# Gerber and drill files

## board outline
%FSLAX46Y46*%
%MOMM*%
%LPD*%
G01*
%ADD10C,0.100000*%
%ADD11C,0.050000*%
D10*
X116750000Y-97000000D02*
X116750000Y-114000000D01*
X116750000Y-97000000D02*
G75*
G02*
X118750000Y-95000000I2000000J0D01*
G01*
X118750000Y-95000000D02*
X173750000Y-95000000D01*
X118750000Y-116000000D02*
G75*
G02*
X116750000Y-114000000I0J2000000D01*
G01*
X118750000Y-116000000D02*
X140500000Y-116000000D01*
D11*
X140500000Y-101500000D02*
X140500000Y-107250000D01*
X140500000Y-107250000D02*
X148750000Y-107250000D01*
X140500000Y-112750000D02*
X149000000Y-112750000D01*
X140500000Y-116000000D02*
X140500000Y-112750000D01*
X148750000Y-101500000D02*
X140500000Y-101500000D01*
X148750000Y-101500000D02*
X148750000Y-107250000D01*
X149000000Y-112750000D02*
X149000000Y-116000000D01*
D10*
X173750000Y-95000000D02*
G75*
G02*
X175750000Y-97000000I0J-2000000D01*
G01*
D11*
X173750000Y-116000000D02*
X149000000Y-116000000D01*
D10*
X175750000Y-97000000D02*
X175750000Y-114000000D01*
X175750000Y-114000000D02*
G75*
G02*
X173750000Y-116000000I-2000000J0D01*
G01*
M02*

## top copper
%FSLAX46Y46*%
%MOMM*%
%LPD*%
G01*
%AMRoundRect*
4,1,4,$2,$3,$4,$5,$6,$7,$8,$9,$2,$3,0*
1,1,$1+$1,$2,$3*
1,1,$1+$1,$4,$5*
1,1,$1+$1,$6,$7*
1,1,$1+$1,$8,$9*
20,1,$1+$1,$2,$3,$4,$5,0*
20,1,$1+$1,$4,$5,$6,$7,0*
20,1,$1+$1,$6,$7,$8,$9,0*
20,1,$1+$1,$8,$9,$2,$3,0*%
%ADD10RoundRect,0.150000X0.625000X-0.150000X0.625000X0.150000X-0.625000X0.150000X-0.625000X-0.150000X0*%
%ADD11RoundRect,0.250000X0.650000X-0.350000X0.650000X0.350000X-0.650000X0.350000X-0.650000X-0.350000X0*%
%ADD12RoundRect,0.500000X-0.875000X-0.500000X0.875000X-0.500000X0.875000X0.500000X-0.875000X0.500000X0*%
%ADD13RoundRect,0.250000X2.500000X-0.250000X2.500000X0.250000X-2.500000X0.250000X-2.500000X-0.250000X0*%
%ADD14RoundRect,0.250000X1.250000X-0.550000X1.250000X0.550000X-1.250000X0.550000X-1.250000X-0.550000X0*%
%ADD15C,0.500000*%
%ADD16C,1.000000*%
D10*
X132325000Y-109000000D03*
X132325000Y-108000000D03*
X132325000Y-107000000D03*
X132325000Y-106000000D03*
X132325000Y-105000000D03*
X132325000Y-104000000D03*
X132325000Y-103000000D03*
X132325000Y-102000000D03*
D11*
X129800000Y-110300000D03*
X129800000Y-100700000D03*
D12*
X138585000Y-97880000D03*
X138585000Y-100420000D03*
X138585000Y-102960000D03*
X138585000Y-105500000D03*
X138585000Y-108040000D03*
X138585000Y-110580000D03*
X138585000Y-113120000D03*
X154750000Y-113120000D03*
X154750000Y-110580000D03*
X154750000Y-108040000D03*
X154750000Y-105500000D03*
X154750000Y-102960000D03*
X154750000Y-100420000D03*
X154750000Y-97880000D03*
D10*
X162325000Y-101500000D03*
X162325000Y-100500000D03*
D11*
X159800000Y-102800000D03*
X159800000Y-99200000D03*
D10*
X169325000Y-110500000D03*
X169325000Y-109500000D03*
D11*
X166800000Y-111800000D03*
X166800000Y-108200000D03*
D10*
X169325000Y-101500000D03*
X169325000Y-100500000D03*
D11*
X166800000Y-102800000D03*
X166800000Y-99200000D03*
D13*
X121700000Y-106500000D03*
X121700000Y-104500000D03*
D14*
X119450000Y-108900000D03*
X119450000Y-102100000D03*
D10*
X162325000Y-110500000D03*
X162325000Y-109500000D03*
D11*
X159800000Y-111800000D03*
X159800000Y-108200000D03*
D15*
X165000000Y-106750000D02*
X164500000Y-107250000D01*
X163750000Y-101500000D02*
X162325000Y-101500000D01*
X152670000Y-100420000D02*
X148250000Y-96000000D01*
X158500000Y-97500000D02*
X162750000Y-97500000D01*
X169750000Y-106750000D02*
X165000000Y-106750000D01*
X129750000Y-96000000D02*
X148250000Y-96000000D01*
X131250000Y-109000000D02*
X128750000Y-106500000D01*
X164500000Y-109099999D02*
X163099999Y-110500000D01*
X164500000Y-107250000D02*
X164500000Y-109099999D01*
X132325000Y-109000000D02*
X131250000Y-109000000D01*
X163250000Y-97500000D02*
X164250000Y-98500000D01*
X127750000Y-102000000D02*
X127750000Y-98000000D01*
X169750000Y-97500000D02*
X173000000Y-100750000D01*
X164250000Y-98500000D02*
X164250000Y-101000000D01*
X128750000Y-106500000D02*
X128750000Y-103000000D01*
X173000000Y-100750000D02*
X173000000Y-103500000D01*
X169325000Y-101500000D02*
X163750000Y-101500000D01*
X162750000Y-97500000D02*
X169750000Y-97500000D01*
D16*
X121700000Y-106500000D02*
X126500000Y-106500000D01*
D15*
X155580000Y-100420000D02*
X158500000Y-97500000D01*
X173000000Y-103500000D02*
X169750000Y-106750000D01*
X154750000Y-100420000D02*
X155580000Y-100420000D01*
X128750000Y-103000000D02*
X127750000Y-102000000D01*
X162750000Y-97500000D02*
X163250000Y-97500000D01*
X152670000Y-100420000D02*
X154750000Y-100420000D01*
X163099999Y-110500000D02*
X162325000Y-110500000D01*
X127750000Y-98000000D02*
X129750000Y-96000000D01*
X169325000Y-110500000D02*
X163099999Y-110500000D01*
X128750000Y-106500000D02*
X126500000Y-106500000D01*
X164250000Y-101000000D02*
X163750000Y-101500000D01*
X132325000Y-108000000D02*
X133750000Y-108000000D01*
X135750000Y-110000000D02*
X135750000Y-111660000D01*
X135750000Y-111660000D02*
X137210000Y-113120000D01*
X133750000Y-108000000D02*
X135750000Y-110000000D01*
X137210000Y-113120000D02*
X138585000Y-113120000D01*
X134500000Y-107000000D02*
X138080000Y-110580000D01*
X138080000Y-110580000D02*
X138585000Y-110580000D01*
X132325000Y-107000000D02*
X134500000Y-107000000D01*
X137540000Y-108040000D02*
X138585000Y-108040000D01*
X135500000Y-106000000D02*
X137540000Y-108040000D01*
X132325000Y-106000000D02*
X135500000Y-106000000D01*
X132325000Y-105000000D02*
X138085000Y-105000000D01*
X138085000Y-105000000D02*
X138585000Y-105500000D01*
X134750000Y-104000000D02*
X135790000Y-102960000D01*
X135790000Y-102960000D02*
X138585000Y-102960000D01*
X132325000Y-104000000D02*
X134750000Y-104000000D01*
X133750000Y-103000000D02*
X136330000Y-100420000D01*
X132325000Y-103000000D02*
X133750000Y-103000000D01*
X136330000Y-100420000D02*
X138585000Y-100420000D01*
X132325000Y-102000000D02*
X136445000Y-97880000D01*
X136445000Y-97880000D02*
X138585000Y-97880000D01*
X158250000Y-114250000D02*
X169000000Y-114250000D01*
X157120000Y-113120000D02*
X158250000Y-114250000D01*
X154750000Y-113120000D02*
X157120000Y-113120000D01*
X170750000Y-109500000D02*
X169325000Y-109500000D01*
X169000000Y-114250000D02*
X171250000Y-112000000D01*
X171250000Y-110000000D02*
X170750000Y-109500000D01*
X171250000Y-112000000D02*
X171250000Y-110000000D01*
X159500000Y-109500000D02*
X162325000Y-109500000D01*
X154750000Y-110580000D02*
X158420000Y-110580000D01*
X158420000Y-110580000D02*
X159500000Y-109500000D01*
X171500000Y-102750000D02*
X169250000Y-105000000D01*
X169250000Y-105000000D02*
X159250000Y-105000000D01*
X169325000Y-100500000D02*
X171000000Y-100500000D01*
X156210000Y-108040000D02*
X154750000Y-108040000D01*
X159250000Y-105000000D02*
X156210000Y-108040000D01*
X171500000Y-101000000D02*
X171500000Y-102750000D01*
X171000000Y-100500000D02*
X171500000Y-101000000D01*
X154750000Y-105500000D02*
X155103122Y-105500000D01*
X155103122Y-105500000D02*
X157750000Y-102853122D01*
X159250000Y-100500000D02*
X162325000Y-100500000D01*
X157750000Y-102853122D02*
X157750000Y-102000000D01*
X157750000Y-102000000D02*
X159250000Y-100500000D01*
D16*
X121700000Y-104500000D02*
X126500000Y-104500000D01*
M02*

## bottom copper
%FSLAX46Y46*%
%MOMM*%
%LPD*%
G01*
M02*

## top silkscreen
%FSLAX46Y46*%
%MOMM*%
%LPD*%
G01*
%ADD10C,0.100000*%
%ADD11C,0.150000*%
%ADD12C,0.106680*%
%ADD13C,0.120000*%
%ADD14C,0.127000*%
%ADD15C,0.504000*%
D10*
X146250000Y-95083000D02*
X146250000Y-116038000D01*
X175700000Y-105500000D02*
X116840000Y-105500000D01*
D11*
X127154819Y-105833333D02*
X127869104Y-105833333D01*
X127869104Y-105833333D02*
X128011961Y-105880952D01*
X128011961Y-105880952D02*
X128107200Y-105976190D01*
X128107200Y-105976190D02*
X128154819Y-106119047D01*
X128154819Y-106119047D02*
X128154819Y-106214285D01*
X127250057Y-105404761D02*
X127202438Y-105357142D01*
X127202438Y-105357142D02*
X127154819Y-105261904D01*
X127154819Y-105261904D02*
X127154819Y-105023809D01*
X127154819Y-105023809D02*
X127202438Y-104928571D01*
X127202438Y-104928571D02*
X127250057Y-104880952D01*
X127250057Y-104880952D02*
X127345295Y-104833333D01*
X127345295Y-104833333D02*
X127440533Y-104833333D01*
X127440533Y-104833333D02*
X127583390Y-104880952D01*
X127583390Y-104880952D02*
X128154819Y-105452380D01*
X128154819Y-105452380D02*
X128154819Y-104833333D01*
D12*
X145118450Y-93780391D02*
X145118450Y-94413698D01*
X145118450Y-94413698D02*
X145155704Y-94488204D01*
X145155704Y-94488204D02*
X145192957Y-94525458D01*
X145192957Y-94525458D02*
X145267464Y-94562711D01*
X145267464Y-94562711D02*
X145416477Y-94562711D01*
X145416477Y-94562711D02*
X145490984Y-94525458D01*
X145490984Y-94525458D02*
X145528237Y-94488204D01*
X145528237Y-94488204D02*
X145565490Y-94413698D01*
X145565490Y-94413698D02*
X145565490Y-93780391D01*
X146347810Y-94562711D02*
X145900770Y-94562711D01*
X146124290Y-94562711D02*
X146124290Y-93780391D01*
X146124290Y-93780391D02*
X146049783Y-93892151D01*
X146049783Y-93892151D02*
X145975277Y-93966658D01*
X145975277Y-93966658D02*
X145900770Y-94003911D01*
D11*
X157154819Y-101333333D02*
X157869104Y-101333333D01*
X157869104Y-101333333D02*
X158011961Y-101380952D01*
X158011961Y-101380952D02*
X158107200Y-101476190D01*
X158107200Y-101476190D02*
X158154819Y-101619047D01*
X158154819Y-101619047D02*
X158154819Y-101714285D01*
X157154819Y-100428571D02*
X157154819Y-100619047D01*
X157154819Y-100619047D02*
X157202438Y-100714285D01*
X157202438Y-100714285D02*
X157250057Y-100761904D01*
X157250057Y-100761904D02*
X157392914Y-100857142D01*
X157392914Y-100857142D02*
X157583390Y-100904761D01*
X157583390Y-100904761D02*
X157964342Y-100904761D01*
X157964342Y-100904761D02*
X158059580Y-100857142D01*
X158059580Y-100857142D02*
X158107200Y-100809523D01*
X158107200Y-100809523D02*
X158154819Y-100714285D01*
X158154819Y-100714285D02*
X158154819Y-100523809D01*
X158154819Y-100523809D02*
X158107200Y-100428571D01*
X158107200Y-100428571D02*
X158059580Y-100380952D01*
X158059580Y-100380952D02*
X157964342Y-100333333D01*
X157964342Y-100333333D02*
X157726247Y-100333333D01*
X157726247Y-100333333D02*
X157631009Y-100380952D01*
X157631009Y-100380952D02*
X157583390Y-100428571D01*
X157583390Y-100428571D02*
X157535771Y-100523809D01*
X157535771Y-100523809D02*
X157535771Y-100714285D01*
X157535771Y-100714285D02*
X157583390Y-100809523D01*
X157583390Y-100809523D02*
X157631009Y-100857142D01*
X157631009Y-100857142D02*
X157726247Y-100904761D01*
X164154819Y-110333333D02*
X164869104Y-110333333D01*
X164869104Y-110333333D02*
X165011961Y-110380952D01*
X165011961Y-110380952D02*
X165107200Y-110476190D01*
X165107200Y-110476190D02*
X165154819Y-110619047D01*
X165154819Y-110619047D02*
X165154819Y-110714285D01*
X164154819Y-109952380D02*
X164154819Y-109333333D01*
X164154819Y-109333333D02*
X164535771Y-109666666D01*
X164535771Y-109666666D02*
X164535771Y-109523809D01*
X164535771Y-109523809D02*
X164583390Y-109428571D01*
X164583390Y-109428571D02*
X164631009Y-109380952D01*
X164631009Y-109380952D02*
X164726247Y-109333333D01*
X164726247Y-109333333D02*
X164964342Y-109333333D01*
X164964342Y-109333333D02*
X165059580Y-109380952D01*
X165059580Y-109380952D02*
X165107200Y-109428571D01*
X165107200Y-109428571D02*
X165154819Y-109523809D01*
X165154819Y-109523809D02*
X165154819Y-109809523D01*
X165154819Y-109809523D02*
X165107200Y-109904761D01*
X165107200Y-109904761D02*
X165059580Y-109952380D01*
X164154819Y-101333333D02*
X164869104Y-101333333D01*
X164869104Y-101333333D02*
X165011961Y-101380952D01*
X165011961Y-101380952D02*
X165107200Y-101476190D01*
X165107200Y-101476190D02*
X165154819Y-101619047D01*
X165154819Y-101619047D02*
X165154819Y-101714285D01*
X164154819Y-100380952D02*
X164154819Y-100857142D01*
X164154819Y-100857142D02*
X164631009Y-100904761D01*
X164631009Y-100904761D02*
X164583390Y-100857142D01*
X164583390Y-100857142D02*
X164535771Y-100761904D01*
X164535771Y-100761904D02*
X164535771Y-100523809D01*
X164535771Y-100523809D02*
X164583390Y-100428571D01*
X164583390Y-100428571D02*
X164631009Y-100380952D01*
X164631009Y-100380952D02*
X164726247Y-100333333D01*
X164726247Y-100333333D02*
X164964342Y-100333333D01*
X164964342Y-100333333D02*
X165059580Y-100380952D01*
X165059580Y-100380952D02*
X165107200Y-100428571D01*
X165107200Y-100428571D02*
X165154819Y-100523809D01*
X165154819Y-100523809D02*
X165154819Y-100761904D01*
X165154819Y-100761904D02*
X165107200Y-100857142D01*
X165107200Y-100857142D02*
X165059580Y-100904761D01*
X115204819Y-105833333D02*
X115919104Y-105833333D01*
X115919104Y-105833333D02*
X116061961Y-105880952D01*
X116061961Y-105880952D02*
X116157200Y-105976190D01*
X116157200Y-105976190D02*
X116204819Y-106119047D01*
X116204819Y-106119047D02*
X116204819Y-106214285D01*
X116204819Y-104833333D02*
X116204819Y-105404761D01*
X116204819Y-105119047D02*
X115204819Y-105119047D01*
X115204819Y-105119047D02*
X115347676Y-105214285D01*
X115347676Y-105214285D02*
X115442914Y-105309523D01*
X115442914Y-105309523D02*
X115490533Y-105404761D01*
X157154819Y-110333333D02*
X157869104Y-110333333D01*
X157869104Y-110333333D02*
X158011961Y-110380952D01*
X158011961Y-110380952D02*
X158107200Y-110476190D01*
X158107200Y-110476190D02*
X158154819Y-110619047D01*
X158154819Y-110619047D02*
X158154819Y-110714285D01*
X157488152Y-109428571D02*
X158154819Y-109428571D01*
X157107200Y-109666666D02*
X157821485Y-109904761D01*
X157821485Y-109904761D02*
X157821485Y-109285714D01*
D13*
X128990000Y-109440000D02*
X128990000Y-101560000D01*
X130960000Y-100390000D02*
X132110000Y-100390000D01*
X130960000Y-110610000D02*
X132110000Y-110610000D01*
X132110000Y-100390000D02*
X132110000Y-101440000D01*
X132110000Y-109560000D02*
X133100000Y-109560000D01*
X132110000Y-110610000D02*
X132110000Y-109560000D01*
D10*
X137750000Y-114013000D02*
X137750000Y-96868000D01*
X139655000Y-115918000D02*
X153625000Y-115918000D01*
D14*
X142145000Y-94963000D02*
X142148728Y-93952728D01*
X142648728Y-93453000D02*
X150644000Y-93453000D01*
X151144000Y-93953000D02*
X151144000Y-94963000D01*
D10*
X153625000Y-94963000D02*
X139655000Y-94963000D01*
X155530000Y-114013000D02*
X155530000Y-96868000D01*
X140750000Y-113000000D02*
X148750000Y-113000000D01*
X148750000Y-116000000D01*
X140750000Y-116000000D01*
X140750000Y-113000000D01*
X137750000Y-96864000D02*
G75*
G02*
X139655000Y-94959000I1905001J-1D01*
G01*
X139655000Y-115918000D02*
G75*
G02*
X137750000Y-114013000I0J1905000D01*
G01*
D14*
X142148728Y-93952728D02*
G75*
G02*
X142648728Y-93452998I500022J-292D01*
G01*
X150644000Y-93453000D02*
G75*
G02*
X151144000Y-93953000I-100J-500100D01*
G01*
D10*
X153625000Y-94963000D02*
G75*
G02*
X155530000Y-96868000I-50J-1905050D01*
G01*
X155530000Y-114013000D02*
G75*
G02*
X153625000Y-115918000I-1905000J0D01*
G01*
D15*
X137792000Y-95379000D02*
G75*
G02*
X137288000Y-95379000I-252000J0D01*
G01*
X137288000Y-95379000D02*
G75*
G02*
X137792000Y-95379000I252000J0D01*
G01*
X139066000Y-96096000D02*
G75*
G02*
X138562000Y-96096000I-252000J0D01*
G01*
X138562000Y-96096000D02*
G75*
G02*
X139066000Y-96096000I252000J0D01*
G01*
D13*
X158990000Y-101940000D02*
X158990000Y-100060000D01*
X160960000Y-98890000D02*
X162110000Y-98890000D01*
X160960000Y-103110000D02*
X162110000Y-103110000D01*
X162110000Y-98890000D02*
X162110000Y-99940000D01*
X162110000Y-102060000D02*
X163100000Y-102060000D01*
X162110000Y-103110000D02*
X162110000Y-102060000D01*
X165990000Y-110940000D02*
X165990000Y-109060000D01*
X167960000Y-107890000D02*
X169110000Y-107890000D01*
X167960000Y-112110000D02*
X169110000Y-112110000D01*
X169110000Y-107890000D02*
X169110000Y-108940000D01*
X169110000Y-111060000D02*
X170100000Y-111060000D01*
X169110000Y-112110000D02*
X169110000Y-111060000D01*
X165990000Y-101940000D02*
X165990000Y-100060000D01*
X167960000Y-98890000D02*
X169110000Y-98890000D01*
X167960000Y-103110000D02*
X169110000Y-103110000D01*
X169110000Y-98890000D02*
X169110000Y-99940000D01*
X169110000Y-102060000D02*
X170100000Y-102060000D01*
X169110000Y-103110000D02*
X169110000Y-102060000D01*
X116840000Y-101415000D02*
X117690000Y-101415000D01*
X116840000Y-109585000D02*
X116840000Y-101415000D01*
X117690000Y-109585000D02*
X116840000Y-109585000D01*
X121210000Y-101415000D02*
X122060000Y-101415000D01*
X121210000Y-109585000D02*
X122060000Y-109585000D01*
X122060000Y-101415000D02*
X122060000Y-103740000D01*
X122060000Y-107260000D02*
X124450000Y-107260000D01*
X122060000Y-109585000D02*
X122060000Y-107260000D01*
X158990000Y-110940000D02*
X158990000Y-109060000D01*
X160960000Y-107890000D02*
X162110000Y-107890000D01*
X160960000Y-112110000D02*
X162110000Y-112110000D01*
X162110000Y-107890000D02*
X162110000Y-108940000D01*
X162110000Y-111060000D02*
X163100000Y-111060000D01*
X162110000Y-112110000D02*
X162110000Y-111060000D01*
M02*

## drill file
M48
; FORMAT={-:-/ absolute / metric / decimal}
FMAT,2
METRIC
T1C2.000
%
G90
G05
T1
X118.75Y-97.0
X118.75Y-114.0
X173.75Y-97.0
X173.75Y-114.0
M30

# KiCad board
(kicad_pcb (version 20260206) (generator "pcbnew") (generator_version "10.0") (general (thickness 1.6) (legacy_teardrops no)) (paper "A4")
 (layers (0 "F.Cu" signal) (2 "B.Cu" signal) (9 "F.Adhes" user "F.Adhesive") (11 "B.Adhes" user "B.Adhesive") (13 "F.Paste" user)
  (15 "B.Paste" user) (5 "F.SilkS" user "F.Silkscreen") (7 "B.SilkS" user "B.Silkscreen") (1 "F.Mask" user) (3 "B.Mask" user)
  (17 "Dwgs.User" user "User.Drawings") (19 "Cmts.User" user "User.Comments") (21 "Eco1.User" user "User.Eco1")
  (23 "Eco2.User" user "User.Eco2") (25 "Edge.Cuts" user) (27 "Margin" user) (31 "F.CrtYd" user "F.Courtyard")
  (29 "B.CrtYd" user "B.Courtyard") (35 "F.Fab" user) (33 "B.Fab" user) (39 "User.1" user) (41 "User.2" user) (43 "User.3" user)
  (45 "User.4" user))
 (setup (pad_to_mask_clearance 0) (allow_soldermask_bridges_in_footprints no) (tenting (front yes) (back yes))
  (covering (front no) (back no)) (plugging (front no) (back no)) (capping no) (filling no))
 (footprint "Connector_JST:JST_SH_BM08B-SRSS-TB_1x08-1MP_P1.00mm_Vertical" (layer "F.Cu") (at 131 105.5 90)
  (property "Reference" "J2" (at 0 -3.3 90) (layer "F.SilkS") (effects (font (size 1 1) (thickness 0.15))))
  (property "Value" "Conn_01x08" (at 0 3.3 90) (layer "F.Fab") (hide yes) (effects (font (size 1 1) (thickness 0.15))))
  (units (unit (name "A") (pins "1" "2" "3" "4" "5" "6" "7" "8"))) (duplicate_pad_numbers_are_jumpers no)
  (fp_line (start -3.94 -2.01) (end 3.94 -2.01) (stroke (width 0.12) (type solid)) (layer "F.SilkS"))
  (fp_line (start 5.11 -0.04) (end 5.11 1.11) (stroke (width 0.12) (type solid)) (layer "F.SilkS"))
  (fp_line (start -5.11 -0.04) (end -5.11 1.11) (stroke (width 0.12) (type solid)) (layer "F.SilkS"))
  (fp_line (start 5.11 1.11) (end 4.06 1.11) (stroke (width 0.12) (type solid)) (layer "F.SilkS"))
  (fp_line (start -4.06 1.11) (end -4.06 2.1) (stroke (width 0.12) (type solid)) (layer "F.SilkS"))
  (fp_line (start -5.11 1.11) (end -4.06 1.11) (stroke (width 0.12) (type solid)) (layer "F.SilkS"))
  (pad "1" smd roundrect (at -3.5 1.325 90) (size 0.6 1.55) (layers "F.Cu" "F.Mask" "F.Paste") (roundrect_rratio 0.25) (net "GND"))
  (pad "2" smd roundrect (at -2.5 1.325 90) (size 0.6 1.55) (layers "F.Cu" "F.Mask" "F.Paste") (roundrect_rratio 0.25)
   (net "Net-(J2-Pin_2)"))
  (pad "3" smd roundrect (at -1.5 1.325 90) (size 0.6 1.55) (layers "F.Cu" "F.Mask" "F.Paste") (roundrect_rratio 0.25)
   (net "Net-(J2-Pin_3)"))
  (pad "4" smd roundrect (at -0.5 1.325 90) (size 0.6 1.55) (layers "F.Cu" "F.Mask" "F.Paste") (roundrect_rratio 0.25)
   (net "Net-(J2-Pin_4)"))
  (pad "5" smd roundrect (at 0.5 1.325 90) (size 0.6 1.55) (layers "F.Cu" "F.Mask" "F.Paste") (roundrect_rratio 0.25) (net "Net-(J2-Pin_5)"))
  (pad "6" smd roundrect (at 1.5 1.325 90) (size 0.6 1.55) (layers "F.Cu" "F.Mask" "F.Paste") (roundrect_rratio 0.25) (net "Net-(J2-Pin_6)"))
  (pad "7" smd roundrect (at 2.5 1.325 90) (size 0.6 1.55) (layers "F.Cu" "F.Mask" "F.Paste") (roundrect_rratio 0.25) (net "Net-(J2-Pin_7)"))
  (pad "8" smd roundrect (at 3.5 1.325 90) (size 0.6 1.55) (layers "F.Cu" "F.Mask" "F.Paste") (roundrect_rratio 0.25) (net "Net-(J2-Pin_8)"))
  (pad "MP" smd roundrect (at -4.8 -1.2 90) (size 1.2 1.8) (layers "F.Cu" "F.Mask" "F.Paste") (roundrect_rratio 0.208333))
  (pad "MP" smd roundrect (at 4.8 -1.2 90) (size 1.2 1.8) (layers "F.Cu" "F.Mask" "F.Paste") (roundrect_rratio 0.208333)))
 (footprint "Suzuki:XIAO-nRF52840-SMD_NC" (layer "F.Cu") (at 137.75 116)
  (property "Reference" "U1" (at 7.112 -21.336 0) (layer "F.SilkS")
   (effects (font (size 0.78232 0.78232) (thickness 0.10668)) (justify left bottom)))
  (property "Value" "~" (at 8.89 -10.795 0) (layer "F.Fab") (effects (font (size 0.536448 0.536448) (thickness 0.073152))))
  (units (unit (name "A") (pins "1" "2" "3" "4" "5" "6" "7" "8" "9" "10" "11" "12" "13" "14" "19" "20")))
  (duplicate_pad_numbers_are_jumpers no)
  (fp_line (start 0 -1.987) (end 0 -19.132) (stroke (width 0.1) (type solid)) (layer "F.SilkS"))
  (fp_line (start 1.905 -0.082) (end 15.875 -0.082) (stroke (width 0.1) (type solid)) (layer "F.SilkS"))
  (fp_line (start 4.395 -21.037) (end 4.398728 -22.047272) (stroke (width 0.127) (type solid)) (layer "F.SilkS"))
  (fp_line (start 4.898728 -22.547) (end 12.894 -22.547) (stroke (width 0.127) (type solid)) (layer "F.SilkS"))
  (fp_line (start 13.394 -22.047) (end 13.394 -21.037) (stroke (width 0.127) (type solid)) (layer "F.SilkS"))
  (fp_line (start 15.875 -21.037) (end 1.905 -21.037) (stroke (width 0.1) (type solid)) (layer "F.SilkS"))
  (fp_line (start 17.78 -1.987) (end 17.78 -19.132) (stroke (width 0.1) (type solid)) (layer "F.SilkS"))
  (fp_rect (start 3 -3) (end 11 0) (stroke (width 0.1) (type default)) (fill no) (layer "F.SilkS"))
  (fp_arc (start 0 -19.136) (mid 0.557962 -20.483038) (end 1.905 -21.041) (stroke (width 0.1) (type solid)) (layer "F.SilkS"))
  (fp_arc (start 1.905 -0.082) (mid 0.557962 -0.639962) (end 0 -1.987) (stroke (width 0.1) (type solid)) (layer "F.SilkS"))
  (fp_arc (start 4.398728 -22.047272) (mid 4.545276 -22.400644) (end 4.898728 -22.547) (stroke (width 0.127) (type default))
   (layer "F.SilkS"))
  (fp_arc (start 12.894 -22.547) (mid 13.247531 -22.400546) (end 13.394 -22.047) (stroke (width 0.127) (type default)) (layer "F.SilkS"))
  (fp_arc (start 15.875 -21.037) (mid 17.222016 -20.479031) (end 17.78 -19.132) (stroke (width 0.1) (type solid)) (layer "F.SilkS"))
  (fp_arc (start 17.78 -1.987) (mid 17.222038 -0.639961) (end 15.875 -0.082) (stroke (width 0.1) (type solid)) (layer "F.SilkS"))
  (fp_circle (center -0.21 -20.621) (end -0.21 -20.875) (stroke (width 0.5) (type solid)) (fill yes) (layer "F.SilkS"))
  (fp_circle (center 1.064 -19.904) (end 1.064 -20.158) (stroke (width 0.5) (type solid)) (fill yes) (layer "F.SilkS"))
  (pad "1" smd roundrect (at 0.835 -18.12) (size 2.75 2) (layers "F.Cu" "F.Mask" "F.Paste") (roundrect_rratio 0.25) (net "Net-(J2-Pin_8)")
   (solder_mask_margin 0.0508) (thermal_bridge_angle 45))
  (pad "2" smd roundrect (at 0.835 -15.58) (size 2.75 2) (layers "F.Cu" "F.Mask" "F.Paste") (roundrect_rratio 0.25) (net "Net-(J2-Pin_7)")
   (solder_mask_margin 0.0508) (thermal_bridge_angle 45))
  (pad "3" smd roundrect (at 0.835 -13.04) (size 2.75 2) (layers "F.Cu" "F.Mask" "F.Paste") (roundrect_rratio 0.25) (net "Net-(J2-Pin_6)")
   (solder_mask_margin 0.0508) (thermal_bridge_angle 45))
  (pad "4" smd roundrect (at 0.835 -10.5) (size 2.75 2) (layers "F.Cu" "F.Mask" "F.Paste") (roundrect_rratio 0.25) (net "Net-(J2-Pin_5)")
   (solder_mask_margin 0.0508) (thermal_bridge_angle 45))
  (pad "5" smd roundrect (at 0.835 -7.96) (size 2.75 2) (layers "F.Cu" "F.Mask" "F.Paste") (roundrect_rratio 0.25) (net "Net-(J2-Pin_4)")
   (solder_mask_margin 0.0508) (thermal_bridge_angle 45))
  (pad "6" smd roundrect (at 0.835 -5.42) (size 2.75 2) (layers "F.Cu" "F.Mask" "F.Paste") (roundrect_rratio 0.25) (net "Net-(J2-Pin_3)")
   (solder_mask_margin 0.0508) (thermal_bridge_angle 45))
  (pad "7" smd roundrect (at 0.835 -2.88) (size 2.75 2) (layers "F.Cu" "F.Mask" "F.Paste") (roundrect_rratio 0.25) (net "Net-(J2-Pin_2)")
   (solder_mask_margin 0.0508) (thermal_bridge_angle 45))
  (pad "8" smd roundrect (at 17 -2.88) (size 2.75 2) (layers "F.Cu" "F.Mask" "F.Paste") (roundrect_rratio 0.25) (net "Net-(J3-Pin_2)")
   (solder_mask_margin 0.0508) (thermal_bridge_angle 45))
  (pad "9" smd roundrect (at 17 -5.42) (size 2.75 2) (layers "F.Cu" "F.Mask" "F.Paste") (roundrect_rratio 0.25) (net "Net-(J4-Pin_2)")
   (solder_mask_margin 0.0508) (thermal_bridge_angle 45))
  (pad "10" smd roundrect (at 17 -7.96) (size 2.75 2) (layers "F.Cu" "F.Mask" "F.Paste") (roundrect_rratio 0.25) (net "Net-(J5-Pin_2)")
   (solder_mask_margin 0.0508) (thermal_bridge_angle 45))
  (pad "11" smd roundrect (at 17 -10.5) (size 2.75 2) (layers "F.Cu" "F.Mask" "F.Paste") (roundrect_rratio 0.25) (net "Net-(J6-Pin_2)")
   (solder_mask_margin 0.0508) (thermal_bridge_angle 45))
  (pad "12" smd roundrect (at 17 -13.04) (size 2.75 2) (layers "F.Cu" "F.Mask" "F.Paste") (roundrect_rratio 0.25)
   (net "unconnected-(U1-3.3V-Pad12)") (solder_mask_margin 0.0508) (thermal_bridge_angle 45))
  (pad "13" smd roundrect (at 17 -15.58) (size 2.75 2) (layers "F.Cu" "F.Mask" "F.Paste") (roundrect_rratio 0.25) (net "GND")
   (solder_mask_margin 0.0508) (thermal_bridge_angle 45))
  (pad "14" smd roundrect (at 17 -18.12) (size 2.75 2) (layers "F.Cu" "F.Mask" "F.Paste") (roundrect_rratio 0.25)
   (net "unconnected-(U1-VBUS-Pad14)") (solder_mask_margin 0.0508) (thermal_bridge_angle 45))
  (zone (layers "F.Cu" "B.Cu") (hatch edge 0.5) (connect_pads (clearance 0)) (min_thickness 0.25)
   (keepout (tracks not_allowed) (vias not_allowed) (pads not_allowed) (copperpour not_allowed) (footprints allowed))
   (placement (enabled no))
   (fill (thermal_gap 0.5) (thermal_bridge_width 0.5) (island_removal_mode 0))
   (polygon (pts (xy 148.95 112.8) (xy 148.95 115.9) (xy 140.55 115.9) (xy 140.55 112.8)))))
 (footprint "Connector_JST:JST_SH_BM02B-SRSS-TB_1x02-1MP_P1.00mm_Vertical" (layer "F.Cu") (at 161 101 90)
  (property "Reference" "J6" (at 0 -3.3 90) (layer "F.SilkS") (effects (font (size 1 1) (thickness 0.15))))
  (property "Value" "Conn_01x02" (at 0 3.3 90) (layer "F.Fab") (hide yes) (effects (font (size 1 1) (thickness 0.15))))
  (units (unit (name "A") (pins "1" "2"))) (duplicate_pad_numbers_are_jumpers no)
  (fp_line (start -0.94 -2.01) (end 0.94 -2.01) (stroke (width 0.12) (type solid)) (layer "F.SilkS"))
  (fp_line (start 2.11 -0.04) (end 2.11 1.11) (stroke (width 0.12) (type solid)) (layer "F.SilkS"))
  (fp_line (start -2.11 -0.04) (end -2.11 1.11) (stroke (width 0.12) (type solid)) (layer "F.SilkS"))
  (fp_line (start 2.11 1.11) (end 1.06 1.11) (stroke (width 0.12) (type solid)) (layer "F.SilkS"))
  (fp_line (start -1.06 1.11) (end -1.06 2.1) (stroke (width 0.12) (type solid)) (layer "F.SilkS"))
  (fp_line (start -2.11 1.11) (end -1.06 1.11) (stroke (width 0.12) (type solid)) (layer "F.SilkS"))
  (pad "1" smd roundrect (at -0.5 1.325 90) (size 0.6 1.55) (layers "F.Cu" "F.Mask" "F.Paste") (roundrect_rratio 0.25) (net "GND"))
  (pad "2" smd roundrect (at 0.5 1.325 90) (size 0.6 1.55) (layers "F.Cu" "F.Mask" "F.Paste") (roundrect_rratio 0.25) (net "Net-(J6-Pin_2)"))
  (pad "MP" smd roundrect (at -1.8 -1.2 90) (size 1.2 1.8) (layers "F.Cu" "F.Mask" "F.Paste") (roundrect_rratio 0.208333))
  (pad "MP" smd roundrect (at 1.8 -1.2 90) (size 1.2 1.8) (layers "F.Cu" "F.Mask" "F.Paste") (roundrect_rratio 0.208333)))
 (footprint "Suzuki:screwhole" (layer "F.Cu") (at 173.750001 114.000001)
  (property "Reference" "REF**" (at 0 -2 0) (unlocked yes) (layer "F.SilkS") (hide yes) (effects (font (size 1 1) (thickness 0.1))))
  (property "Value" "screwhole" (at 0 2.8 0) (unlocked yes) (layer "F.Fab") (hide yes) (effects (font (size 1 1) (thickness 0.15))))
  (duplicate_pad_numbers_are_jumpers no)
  (pad "" np_thru_hole circle (at 0 0) (size 2 2) (drill 2) (layers "*.Cu" "*.Mask"))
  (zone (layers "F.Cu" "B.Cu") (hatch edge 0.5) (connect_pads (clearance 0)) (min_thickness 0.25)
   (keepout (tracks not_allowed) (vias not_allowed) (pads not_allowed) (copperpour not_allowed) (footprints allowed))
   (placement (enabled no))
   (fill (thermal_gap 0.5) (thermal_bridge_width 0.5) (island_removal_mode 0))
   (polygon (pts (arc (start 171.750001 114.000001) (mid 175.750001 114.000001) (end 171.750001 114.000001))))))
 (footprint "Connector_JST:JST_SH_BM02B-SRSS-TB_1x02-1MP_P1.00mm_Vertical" (layer "F.Cu") (at 168 110 90)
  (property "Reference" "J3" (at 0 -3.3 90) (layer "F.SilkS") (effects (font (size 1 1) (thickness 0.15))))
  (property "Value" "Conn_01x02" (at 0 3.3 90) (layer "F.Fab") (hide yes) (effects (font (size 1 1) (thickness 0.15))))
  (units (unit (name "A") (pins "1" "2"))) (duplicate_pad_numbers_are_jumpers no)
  (fp_line (start -0.94 -2.01) (end 0.94 -2.01) (stroke (width 0.12) (type solid)) (layer "F.SilkS"))
  (fp_line (start 2.11 -0.04) (end 2.11 1.11) (stroke (width 0.12) (type solid)) (layer "F.SilkS"))
  (fp_line (start -2.11 -0.04) (end -2.11 1.11) (stroke (width 0.12) (type solid)) (layer "F.SilkS"))
  (fp_line (start 2.11 1.11) (end 1.06 1.11) (stroke (width 0.12) (type solid)) (layer "F.SilkS"))
  (fp_line (start -1.06 1.11) (end -1.06 2.1) (stroke (width 0.12) (type solid)) (layer "F.SilkS"))
  (fp_line (start -2.11 1.11) (end -1.06 1.11) (stroke (width 0.12) (type solid)) (layer "F.SilkS"))
  (pad "1" smd roundrect (at -0.5 1.325 90) (size 0.6 1.55) (layers "F.Cu" "F.Mask" "F.Paste") (roundrect_rratio 0.25) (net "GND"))
  (pad "2" smd roundrect (at 0.5 1.325 90) (size 0.6 1.55) (layers "F.Cu" "F.Mask" "F.Paste") (roundrect_rratio 0.25) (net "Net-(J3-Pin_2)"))
  (pad "MP" smd roundrect (at -1.8 -1.2 90) (size 1.2 1.8) (layers "F.Cu" "F.Mask" "F.Paste") (roundrect_rratio 0.208333))
  (pad "MP" smd roundrect (at 1.8 -1.2 90) (size 1.2 1.8) (layers "F.Cu" "F.Mask" "F.Paste") (roundrect_rratio 0.208333)))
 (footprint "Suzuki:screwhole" (layer "F.Cu") (at 118.749999 96.999999)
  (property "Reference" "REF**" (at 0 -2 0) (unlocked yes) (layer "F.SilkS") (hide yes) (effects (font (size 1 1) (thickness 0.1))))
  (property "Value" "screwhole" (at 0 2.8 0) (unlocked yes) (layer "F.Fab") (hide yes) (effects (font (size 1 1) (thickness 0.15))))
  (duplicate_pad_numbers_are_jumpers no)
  (pad "" np_thru_hole circle (at 0 0) (size 2 2) (drill 2) (layers "*.Cu" "*.Mask"))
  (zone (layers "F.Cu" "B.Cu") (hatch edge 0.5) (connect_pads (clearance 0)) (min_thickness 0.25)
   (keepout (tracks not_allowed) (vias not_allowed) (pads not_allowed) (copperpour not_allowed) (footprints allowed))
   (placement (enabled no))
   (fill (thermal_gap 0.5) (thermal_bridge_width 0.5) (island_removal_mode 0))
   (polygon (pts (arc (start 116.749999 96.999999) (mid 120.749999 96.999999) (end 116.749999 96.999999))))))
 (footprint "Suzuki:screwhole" (layer "F.Cu") (at 173.750001 96.999999)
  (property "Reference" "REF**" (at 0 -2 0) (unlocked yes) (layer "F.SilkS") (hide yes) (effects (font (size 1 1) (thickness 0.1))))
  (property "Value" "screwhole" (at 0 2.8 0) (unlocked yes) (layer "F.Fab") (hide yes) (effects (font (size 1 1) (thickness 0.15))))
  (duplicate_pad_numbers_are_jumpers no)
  (pad "" np_thru_hole circle (at 0 0) (size 2 2) (drill 2) (layers "*.Cu" "*.Mask"))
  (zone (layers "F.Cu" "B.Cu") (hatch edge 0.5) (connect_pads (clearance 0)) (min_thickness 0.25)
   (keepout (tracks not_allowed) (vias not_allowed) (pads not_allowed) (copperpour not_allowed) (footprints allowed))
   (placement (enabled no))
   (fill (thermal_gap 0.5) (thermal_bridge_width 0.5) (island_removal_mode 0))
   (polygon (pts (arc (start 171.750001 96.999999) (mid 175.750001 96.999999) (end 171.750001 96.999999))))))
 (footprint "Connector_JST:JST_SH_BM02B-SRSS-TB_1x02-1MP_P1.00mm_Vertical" (layer "F.Cu") (at 168 101 90)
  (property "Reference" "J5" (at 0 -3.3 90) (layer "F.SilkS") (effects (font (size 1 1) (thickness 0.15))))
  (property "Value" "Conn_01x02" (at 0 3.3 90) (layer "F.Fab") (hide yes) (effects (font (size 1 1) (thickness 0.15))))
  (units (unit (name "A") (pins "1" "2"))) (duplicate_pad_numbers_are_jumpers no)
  (fp_line (start -0.94 -2.01) (end 0.94 -2.01) (stroke (width 0.12) (type solid)) (layer "F.SilkS"))
  (fp_line (start 2.11 -0.04) (end 2.11 1.11) (stroke (width 0.12) (type solid)) (layer "F.SilkS"))
  (fp_line (start -2.11 -0.04) (end -2.11 1.11) (stroke (width 0.12) (type solid)) (layer "F.SilkS"))
  (fp_line (start 2.11 1.11) (end 1.06 1.11) (stroke (width 0.12) (type solid)) (layer "F.SilkS"))
  (fp_line (start -1.06 1.11) (end -1.06 2.1) (stroke (width 0.12) (type solid)) (layer "F.SilkS"))
  (fp_line (start -2.11 1.11) (end -1.06 1.11) (stroke (width 0.12) (type solid)) (layer "F.SilkS"))
  (pad "1" smd roundrect (at -0.5 1.325 90) (size 0.6 1.55) (layers "F.Cu" "F.Mask" "F.Paste") (roundrect_rratio 0.25) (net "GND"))
  (pad "2" smd roundrect (at 0.5 1.325 90) (size 0.6 1.55) (layers "F.Cu" "F.Mask" "F.Paste") (roundrect_rratio 0.25) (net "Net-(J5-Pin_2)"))
  (pad "MP" smd roundrect (at -1.8 -1.2 90) (size 1.2 1.8) (layers "F.Cu" "F.Mask" "F.Paste") (roundrect_rratio 0.208333))
  (pad "MP" smd roundrect (at 1.8 -1.2 90) (size 1.2 1.8) (layers "F.Cu" "F.Mask" "F.Paste") (roundrect_rratio 0.208333)))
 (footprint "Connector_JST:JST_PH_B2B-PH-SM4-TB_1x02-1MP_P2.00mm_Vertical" (layer "F.Cu") (at 121.2 105.5 90)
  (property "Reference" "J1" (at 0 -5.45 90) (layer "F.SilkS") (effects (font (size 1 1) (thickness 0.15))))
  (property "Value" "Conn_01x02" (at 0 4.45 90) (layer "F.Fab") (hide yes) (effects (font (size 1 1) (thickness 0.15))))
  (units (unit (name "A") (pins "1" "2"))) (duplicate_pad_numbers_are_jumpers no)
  (fp_line (start 4.085 -4.36) (end 4.085 -3.51) (stroke (width 0.12) (type solid)) (layer "F.SilkS"))
  (fp_line (start -4.085 -4.36) (end 4.085 -4.36) (stroke (width 0.12) (type solid)) (layer "F.SilkS"))
  (fp_line (start -4.085 -3.51) (end -4.085 -4.36) (stroke (width 0.12) (type solid)) (layer "F.SilkS"))
  (fp_line (start 4.085 0.01) (end 4.085 0.86) (stroke (width 0.12) (type solid)) (layer "F.SilkS"))
  (fp_line (start -4.085 0.01) (end -4.085 0.86) (stroke (width 0.12) (type solid)) (layer "F.SilkS"))
  (fp_line (start 4.085 0.86) (end 1.76 0.86) (stroke (width 0.12) (type solid)) (layer "F.SilkS"))
  (fp_line (start -1.76 0.86) (end -1.76 3.25) (stroke (width 0.12) (type solid)) (layer "F.SilkS"))
  (fp_line (start -4.085 0.86) (end -1.76 0.86) (stroke (width 0.12) (type solid)) (layer "F.SilkS"))
  (pad "1" smd roundrect (at -1 0.5 90) (size 1 5.5) (layers "F.Cu" "F.Mask" "F.Paste") (roundrect_rratio 0.25) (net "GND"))
  (pad "2" smd roundrect (at 1 0.5 90) (size 1 5.5) (layers "F.Cu" "F.Mask" "F.Paste") (roundrect_rratio 0.25) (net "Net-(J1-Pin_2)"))
  (pad "MP" smd roundrect (at -3.4 -1.75 90) (size 1.6 3) (layers "F.Cu" "F.Mask" "F.Paste") (roundrect_rratio 0.15625))
  (pad "MP" smd roundrect (at 3.4 -1.75 90) (size 1.6 3) (layers "F.Cu" "F.Mask" "F.Paste") (roundrect_rratio 0.15625)))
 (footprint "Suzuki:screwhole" (layer "F.Cu") (at 118.749999 114.000001)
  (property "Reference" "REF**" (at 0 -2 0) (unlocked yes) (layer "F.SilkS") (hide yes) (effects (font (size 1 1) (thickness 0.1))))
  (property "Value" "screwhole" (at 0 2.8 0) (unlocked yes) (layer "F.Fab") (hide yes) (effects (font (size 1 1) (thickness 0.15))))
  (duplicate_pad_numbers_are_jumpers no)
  (pad "" np_thru_hole circle (at 0 0) (size 2 2) (drill 2) (layers "*.Cu" "*.Mask"))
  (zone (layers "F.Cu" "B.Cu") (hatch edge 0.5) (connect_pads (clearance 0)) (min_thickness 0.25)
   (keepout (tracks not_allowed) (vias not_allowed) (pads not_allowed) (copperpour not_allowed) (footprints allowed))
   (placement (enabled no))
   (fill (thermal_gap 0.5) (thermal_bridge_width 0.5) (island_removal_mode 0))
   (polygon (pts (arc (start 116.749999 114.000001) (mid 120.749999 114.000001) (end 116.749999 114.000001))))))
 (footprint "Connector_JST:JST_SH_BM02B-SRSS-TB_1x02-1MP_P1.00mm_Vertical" (layer "F.Cu") (at 161 110 90)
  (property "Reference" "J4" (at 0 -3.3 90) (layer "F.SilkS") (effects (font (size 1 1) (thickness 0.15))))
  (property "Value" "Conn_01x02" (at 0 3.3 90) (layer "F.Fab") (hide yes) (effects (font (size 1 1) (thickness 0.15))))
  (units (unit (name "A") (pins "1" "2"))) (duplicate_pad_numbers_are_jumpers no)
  (fp_line (start -0.94 -2.01) (end 0.94 -2.01) (stroke (width 0.12) (type solid)) (layer "F.SilkS"))
  (fp_line (start 2.11 -0.04) (end 2.11 1.11) (stroke (width 0.12) (type solid)) (layer "F.SilkS"))
  (fp_line (start -2.11 -0.04) (end -2.11 1.11) (stroke (width 0.12) (type solid)) (layer "F.SilkS"))
  (fp_line (start 2.11 1.11) (end 1.06 1.11) (stroke (width 0.12) (type solid)) (layer "F.SilkS"))
  (fp_line (start -1.06 1.11) (end -1.06 2.1) (stroke (width 0.12) (type solid)) (layer "F.SilkS"))
  (fp_line (start -2.11 1.11) (end -1.06 1.11) (stroke (width 0.12) (type solid)) (layer "F.SilkS"))
  (pad "1" smd roundrect (at -0.5 1.325 90) (size 0.6 1.55) (layers "F.Cu" "F.Mask" "F.Paste") (roundrect_rratio 0.25) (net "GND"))
  (pad "2" smd roundrect (at 0.5 1.325 90) (size 0.6 1.55) (layers "F.Cu" "F.Mask" "F.Paste") (roundrect_rratio 0.25) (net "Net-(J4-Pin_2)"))
  (pad "MP" smd roundrect (at -1.8 -1.2 90) (size 1.2 1.8) (layers "F.Cu" "F.Mask" "F.Paste") (roundrect_rratio 0.208333))
  (pad "MP" smd roundrect (at 1.8 -1.2 90) (size 1.2 1.8) (layers "F.Cu" "F.Mask" "F.Paste") (roundrect_rratio 0.208333)))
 (gr_line (start 146.25 95.083) (end 146.25 116.038) (stroke (width 0.1) (type solid)) (layer "F.SilkS"))
 (gr_line (start 175.7 105.5) (end 116.84 105.5) (stroke (width 0.1) (type solid)) (layer "F.SilkS"))
 (gr_line (start 116.75 97) (end 116.75 114) (stroke (width 0.1) (type solid)) (layer "Edge.Cuts"))
 (gr_arc (start 116.75 97) (mid 117.335786 95.585786) (end 118.75 95) (stroke (width 0.1) (type default)) (layer "Edge.Cuts"))
 (gr_line (start 118.75 95) (end 173.75 95) (stroke (width 0.1) (type solid)) (layer "Edge.Cuts"))
 (gr_arc (start 118.75 116) (mid 117.335786 115.414214) (end 116.75 114) (stroke (width 0.1) (type default)) (layer "Edge.Cuts"))
 (gr_line (start 118.75 116) (end 140.5 116) (stroke (width 0.1) (type solid)) (layer "Edge.Cuts"))
 (gr_line (start 140.5 101.5) (end 140.5 107.25) (stroke (width 0.05) (type default)) (layer "Edge.Cuts"))
 (gr_line (start 140.5 107.25) (end 148.75 107.25) (stroke (width 0.05) (type default)) (layer "Edge.Cuts"))
 (gr_line (start 140.5 112.75) (end 149 112.75) (stroke (width 0.05) (type default)) (layer "Edge.Cuts"))
 (gr_line (start 140.5 116) (end 140.5 112.75) (stroke (width 0.05) (type default)) (layer "Edge.Cuts"))
 (gr_line (start 148.75 101.5) (end 140.5 101.5) (stroke (width 0.05) (type default)) (layer "Edge.Cuts"))
 (gr_line (start 148.75 101.5) (end 148.75 107.25) (stroke (width 0.05) (type default)) (layer "Edge.Cuts"))
 (gr_line (start 149 112.75) (end 149 116) (stroke (width 0.05) (type default)) (layer "Edge.Cuts"))
 (gr_arc (start 173.75 95) (mid 175.164214 95.585786) (end 175.75 97) (stroke (width 0.1) (type default)) (layer "Edge.Cuts"))
 (gr_line (start 173.75 116) (end 149 116) (stroke (width 0.05) (type default)) (layer "Edge.Cuts"))
 (gr_line (start 175.75 97) (end 175.75 114) (stroke (width 0.1) (type solid)) (layer "Edge.Cuts"))
 (gr_arc (start 175.75 114) (mid 175.164214 115.414214) (end 173.75 116) (stroke (width 0.1) (type default)) (layer "Edge.Cuts"))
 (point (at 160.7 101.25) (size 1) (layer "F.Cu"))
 (segment (start 165 106.75) (end 164.5 107.25) (width 0.5) (layer "F.Cu") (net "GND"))
 (segment (start 163.75 101.5) (end 162.325 101.5) (width 0.5) (layer "F.Cu") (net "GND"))
 (segment (start 152.67 100.42) (end 148.25 96) (width 0.5) (layer "F.Cu") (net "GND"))
 (segment (start 158.5 97.5) (end 162.75 97.5) (width 0.5) (layer "F.Cu") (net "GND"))
 (segment (start 169.75 106.75) (end 165 106.75) (width 0.5) (layer "F.Cu") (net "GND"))
 (segment (start 129.75 96) (end 148.25 96) (width 0.5) (layer "F.Cu") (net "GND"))
 (segment (start 131.25 109) (end 128.75 106.5) (width 0.5) (layer "F.Cu") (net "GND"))
 (segment (start 164.5 109.099999) (end 163.099999 110.5) (width 0.5) (layer "F.Cu") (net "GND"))
 (segment (start 164.5 107.25) (end 164.5 109.099999) (width 0.5) (layer "F.Cu") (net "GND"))
 (segment (start 132.325 109) (end 131.25 109) (width 0.5) (layer "F.Cu") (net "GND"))
 (segment (start 163.25 97.5) (end 164.25 98.5) (width 0.5) (layer "F.Cu") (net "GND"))
 (segment (start 127.75 102) (end 127.75 98) (width 0.5) (layer "F.Cu") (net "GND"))
 (segment (start 169.75 97.5) (end 173 100.75) (width 0.5) (layer "F.Cu") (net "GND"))
 (segment (start 164.25 98.5) (end 164.25 101) (width 0.5) (layer "F.Cu") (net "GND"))
 (segment (start 128.75 106.5) (end 128.75 103) (width 0.5) (layer "F.Cu") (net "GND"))
 (segment (start 173 100.75) (end 173 103.5) (width 0.5) (layer "F.Cu") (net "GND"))
 (segment (start 169.325 101.5) (end 163.75 101.5) (width 0.5) (layer "F.Cu") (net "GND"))
 (segment (start 162.75 97.5) (end 169.75 97.5) (width 0.5) (layer "F.Cu") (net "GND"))
 (segment (start 121.7 106.5) (end 126.5 106.5) (width 1) (layer "F.Cu") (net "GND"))
 (segment (start 155.58 100.42) (end 158.5 97.5) (width 0.5) (layer "F.Cu") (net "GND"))
 (segment (start 173 103.5) (end 169.75 106.75) (width 0.5) (layer "F.Cu") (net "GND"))
 (segment (start 154.75 100.42) (end 155.58 100.42) (width 0.5) (layer "F.Cu") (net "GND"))
 (segment (start 128.75 103) (end 127.75 102) (width 0.5) (layer "F.Cu") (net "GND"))
 (segment (start 162.75 97.5) (end 163.25 97.5) (width 0.5) (layer "F.Cu") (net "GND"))
 (segment (start 152.67 100.42) (end 154.75 100.42) (width 0.5) (layer "F.Cu") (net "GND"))
 (segment (start 163.099999 110.5) (end 162.325 110.5) (width 0.5) (layer "F.Cu") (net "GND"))
 (segment (start 127.75 98) (end 129.75 96) (width 0.5) (layer "F.Cu") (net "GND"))
 (segment (start 169.325 110.5) (end 163.099999 110.5) (width 0.5) (layer "F.Cu") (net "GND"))
 (segment (start 128.75 106.5) (end 126.5 106.5) (width 0.5) (layer "F.Cu") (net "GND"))
 (segment (start 164.25 101) (end 163.75 101.5) (width 0.5) (layer "F.Cu") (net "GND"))
 (segment (start 132.325 108) (end 133.75 108) (width 0.5) (layer "F.Cu") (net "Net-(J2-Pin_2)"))
 (segment (start 135.75 110) (end 135.75 111.66) (width 0.5) (layer "F.Cu") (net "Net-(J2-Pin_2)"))
 (segment (start 135.75 111.66) (end 137.21 113.12) (width 0.5) (layer "F.Cu") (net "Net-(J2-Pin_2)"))
 (segment (start 133.75 108) (end 135.75 110) (width 0.5) (layer "F.Cu") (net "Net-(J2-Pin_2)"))
 (segment (start 137.21 113.12) (end 138.585 113.12) (width 0.5) (layer "F.Cu") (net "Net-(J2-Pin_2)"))
 (segment (start 134.5 107) (end 138.08 110.58) (width 0.5) (layer "F.Cu") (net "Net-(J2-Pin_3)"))
 (segment (start 138.08 110.58) (end 138.585 110.58) (width 0.5) (layer "F.Cu") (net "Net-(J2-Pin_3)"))
 (segment (start 132.325 107) (end 134.5 107) (width 0.5) (layer "F.Cu") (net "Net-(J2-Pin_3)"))
 (segment (start 137.54 108.04) (end 138.585 108.04) (width 0.5) (layer "F.Cu") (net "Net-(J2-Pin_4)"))
 (segment (start 135.5 106) (end 137.54 108.04) (width 0.5) (layer "F.Cu") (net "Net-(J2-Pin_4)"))
 (segment (start 132.325 106) (end 135.5 106) (width 0.5) (layer "F.Cu") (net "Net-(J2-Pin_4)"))
 (segment (start 132.325 105) (end 138.085 105) (width 0.5) (layer "F.Cu") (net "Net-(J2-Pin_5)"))
 (segment (start 138.085 105) (end 138.585 105.5) (width 0.5) (layer "F.Cu") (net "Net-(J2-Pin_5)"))
 (segment (start 134.75 104) (end 135.79 102.96) (width 0.5) (layer "F.Cu") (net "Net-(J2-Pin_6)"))
 (segment (start 135.79 102.96) (end 138.585 102.96) (width 0.5) (layer "F.Cu") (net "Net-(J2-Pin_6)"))
 (segment (start 132.325 104) (end 134.75 104) (width 0.5) (layer "F.Cu") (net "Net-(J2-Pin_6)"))
 (segment (start 133.75 103) (end 136.33 100.42) (width 0.5) (layer "F.Cu") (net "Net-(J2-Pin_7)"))
 (segment (start 132.325 103) (end 133.75 103) (width 0.5) (layer "F.Cu") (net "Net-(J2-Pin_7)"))
 (segment (start 136.33 100.42) (end 138.585 100.42) (width 0.5) (layer "F.Cu") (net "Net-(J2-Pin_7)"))
 (segment (start 132.325 102) (end 136.445 97.88) (width 0.5) (layer "F.Cu") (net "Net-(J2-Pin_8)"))
 (segment (start 136.445 97.88) (end 138.585 97.88) (width 0.5) (layer "F.Cu") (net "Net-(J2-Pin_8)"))
 (segment (start 158.25 114.25) (end 169 114.25) (width 0.5) (layer "F.Cu") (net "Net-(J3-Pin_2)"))
 (segment (start 157.12 113.12) (end 158.25 114.25) (width 0.5) (layer "F.Cu") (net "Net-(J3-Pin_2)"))
 (segment (start 154.75 113.12) (end 157.12 113.12) (width 0.5) (layer "F.Cu") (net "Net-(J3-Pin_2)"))
 (segment (start 170.75 109.5) (end 169.325 109.5) (width 0.5) (layer "F.Cu") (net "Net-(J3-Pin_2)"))
 (segment (start 169 114.25) (end 171.25 112) (width 0.5) (layer "F.Cu") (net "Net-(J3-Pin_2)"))
 (segment (start 171.25 110) (end 170.75 109.5) (width 0.5) (layer "F.Cu") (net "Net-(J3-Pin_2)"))
 (segment (start 171.25 112) (end 171.25 110) (width 0.5) (layer "F.Cu") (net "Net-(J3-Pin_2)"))
 (segment (start 159.5 109.5) (end 162.325 109.5) (width 0.5) (layer "F.Cu") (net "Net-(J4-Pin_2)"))
 (segment (start 154.75 110.58) (end 158.42 110.58) (width 0.5) (layer "F.Cu") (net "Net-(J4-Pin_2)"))
 (segment (start 158.42 110.58) (end 159.5 109.5) (width 0.5) (layer "F.Cu") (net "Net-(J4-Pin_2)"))
 (segment (start 171.5 102.75) (end 169.25 105) (width 0.5) (layer "F.Cu") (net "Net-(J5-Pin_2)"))
 (segment (start 169.25 105) (end 159.25 105) (width 0.5) (layer "F.Cu") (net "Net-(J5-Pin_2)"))
 (segment (start 169.325 100.5) (end 171 100.5) (width 0.5) (layer "F.Cu") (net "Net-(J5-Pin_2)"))
 (segment (start 156.21 108.04) (end 154.75 108.04) (width 0.5) (layer "F.Cu") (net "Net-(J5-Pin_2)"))
 (segment (start 159.25 105) (end 156.21 108.04) (width 0.5) (layer "F.Cu") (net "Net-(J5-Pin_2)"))
 (segment (start 171.5 101) (end 171.5 102.75) (width 0.5) (layer "F.Cu") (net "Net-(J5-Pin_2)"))
 (segment (start 171 100.5) (end 171.5 101) (width 0.5) (layer "F.Cu") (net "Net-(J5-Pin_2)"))
 (segment (start 154.75 105.5) (end 155.103122 105.5) (width 0.5) (layer "F.Cu") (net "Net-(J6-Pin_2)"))
 (segment (start 155.103122 105.5) (end 157.75 102.853122) (width 0.5) (layer "F.Cu") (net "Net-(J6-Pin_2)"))
 (segment (start 159.25 100.5) (end 162.325 100.5) (width 0.5) (layer "F.Cu") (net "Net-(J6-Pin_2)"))
 (segment (start 157.75 102.853122) (end 157.75 102) (width 0.5) (layer "F.Cu") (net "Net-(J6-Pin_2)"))
 (segment (start 157.75 102) (end 159.25 100.5) (width 0.5) (layer "F.Cu") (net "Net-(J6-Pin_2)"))
 (segment (start 121.7 104.5) (end 126.5 104.5) (width 1) (layer "F.Cu") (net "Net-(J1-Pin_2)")))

